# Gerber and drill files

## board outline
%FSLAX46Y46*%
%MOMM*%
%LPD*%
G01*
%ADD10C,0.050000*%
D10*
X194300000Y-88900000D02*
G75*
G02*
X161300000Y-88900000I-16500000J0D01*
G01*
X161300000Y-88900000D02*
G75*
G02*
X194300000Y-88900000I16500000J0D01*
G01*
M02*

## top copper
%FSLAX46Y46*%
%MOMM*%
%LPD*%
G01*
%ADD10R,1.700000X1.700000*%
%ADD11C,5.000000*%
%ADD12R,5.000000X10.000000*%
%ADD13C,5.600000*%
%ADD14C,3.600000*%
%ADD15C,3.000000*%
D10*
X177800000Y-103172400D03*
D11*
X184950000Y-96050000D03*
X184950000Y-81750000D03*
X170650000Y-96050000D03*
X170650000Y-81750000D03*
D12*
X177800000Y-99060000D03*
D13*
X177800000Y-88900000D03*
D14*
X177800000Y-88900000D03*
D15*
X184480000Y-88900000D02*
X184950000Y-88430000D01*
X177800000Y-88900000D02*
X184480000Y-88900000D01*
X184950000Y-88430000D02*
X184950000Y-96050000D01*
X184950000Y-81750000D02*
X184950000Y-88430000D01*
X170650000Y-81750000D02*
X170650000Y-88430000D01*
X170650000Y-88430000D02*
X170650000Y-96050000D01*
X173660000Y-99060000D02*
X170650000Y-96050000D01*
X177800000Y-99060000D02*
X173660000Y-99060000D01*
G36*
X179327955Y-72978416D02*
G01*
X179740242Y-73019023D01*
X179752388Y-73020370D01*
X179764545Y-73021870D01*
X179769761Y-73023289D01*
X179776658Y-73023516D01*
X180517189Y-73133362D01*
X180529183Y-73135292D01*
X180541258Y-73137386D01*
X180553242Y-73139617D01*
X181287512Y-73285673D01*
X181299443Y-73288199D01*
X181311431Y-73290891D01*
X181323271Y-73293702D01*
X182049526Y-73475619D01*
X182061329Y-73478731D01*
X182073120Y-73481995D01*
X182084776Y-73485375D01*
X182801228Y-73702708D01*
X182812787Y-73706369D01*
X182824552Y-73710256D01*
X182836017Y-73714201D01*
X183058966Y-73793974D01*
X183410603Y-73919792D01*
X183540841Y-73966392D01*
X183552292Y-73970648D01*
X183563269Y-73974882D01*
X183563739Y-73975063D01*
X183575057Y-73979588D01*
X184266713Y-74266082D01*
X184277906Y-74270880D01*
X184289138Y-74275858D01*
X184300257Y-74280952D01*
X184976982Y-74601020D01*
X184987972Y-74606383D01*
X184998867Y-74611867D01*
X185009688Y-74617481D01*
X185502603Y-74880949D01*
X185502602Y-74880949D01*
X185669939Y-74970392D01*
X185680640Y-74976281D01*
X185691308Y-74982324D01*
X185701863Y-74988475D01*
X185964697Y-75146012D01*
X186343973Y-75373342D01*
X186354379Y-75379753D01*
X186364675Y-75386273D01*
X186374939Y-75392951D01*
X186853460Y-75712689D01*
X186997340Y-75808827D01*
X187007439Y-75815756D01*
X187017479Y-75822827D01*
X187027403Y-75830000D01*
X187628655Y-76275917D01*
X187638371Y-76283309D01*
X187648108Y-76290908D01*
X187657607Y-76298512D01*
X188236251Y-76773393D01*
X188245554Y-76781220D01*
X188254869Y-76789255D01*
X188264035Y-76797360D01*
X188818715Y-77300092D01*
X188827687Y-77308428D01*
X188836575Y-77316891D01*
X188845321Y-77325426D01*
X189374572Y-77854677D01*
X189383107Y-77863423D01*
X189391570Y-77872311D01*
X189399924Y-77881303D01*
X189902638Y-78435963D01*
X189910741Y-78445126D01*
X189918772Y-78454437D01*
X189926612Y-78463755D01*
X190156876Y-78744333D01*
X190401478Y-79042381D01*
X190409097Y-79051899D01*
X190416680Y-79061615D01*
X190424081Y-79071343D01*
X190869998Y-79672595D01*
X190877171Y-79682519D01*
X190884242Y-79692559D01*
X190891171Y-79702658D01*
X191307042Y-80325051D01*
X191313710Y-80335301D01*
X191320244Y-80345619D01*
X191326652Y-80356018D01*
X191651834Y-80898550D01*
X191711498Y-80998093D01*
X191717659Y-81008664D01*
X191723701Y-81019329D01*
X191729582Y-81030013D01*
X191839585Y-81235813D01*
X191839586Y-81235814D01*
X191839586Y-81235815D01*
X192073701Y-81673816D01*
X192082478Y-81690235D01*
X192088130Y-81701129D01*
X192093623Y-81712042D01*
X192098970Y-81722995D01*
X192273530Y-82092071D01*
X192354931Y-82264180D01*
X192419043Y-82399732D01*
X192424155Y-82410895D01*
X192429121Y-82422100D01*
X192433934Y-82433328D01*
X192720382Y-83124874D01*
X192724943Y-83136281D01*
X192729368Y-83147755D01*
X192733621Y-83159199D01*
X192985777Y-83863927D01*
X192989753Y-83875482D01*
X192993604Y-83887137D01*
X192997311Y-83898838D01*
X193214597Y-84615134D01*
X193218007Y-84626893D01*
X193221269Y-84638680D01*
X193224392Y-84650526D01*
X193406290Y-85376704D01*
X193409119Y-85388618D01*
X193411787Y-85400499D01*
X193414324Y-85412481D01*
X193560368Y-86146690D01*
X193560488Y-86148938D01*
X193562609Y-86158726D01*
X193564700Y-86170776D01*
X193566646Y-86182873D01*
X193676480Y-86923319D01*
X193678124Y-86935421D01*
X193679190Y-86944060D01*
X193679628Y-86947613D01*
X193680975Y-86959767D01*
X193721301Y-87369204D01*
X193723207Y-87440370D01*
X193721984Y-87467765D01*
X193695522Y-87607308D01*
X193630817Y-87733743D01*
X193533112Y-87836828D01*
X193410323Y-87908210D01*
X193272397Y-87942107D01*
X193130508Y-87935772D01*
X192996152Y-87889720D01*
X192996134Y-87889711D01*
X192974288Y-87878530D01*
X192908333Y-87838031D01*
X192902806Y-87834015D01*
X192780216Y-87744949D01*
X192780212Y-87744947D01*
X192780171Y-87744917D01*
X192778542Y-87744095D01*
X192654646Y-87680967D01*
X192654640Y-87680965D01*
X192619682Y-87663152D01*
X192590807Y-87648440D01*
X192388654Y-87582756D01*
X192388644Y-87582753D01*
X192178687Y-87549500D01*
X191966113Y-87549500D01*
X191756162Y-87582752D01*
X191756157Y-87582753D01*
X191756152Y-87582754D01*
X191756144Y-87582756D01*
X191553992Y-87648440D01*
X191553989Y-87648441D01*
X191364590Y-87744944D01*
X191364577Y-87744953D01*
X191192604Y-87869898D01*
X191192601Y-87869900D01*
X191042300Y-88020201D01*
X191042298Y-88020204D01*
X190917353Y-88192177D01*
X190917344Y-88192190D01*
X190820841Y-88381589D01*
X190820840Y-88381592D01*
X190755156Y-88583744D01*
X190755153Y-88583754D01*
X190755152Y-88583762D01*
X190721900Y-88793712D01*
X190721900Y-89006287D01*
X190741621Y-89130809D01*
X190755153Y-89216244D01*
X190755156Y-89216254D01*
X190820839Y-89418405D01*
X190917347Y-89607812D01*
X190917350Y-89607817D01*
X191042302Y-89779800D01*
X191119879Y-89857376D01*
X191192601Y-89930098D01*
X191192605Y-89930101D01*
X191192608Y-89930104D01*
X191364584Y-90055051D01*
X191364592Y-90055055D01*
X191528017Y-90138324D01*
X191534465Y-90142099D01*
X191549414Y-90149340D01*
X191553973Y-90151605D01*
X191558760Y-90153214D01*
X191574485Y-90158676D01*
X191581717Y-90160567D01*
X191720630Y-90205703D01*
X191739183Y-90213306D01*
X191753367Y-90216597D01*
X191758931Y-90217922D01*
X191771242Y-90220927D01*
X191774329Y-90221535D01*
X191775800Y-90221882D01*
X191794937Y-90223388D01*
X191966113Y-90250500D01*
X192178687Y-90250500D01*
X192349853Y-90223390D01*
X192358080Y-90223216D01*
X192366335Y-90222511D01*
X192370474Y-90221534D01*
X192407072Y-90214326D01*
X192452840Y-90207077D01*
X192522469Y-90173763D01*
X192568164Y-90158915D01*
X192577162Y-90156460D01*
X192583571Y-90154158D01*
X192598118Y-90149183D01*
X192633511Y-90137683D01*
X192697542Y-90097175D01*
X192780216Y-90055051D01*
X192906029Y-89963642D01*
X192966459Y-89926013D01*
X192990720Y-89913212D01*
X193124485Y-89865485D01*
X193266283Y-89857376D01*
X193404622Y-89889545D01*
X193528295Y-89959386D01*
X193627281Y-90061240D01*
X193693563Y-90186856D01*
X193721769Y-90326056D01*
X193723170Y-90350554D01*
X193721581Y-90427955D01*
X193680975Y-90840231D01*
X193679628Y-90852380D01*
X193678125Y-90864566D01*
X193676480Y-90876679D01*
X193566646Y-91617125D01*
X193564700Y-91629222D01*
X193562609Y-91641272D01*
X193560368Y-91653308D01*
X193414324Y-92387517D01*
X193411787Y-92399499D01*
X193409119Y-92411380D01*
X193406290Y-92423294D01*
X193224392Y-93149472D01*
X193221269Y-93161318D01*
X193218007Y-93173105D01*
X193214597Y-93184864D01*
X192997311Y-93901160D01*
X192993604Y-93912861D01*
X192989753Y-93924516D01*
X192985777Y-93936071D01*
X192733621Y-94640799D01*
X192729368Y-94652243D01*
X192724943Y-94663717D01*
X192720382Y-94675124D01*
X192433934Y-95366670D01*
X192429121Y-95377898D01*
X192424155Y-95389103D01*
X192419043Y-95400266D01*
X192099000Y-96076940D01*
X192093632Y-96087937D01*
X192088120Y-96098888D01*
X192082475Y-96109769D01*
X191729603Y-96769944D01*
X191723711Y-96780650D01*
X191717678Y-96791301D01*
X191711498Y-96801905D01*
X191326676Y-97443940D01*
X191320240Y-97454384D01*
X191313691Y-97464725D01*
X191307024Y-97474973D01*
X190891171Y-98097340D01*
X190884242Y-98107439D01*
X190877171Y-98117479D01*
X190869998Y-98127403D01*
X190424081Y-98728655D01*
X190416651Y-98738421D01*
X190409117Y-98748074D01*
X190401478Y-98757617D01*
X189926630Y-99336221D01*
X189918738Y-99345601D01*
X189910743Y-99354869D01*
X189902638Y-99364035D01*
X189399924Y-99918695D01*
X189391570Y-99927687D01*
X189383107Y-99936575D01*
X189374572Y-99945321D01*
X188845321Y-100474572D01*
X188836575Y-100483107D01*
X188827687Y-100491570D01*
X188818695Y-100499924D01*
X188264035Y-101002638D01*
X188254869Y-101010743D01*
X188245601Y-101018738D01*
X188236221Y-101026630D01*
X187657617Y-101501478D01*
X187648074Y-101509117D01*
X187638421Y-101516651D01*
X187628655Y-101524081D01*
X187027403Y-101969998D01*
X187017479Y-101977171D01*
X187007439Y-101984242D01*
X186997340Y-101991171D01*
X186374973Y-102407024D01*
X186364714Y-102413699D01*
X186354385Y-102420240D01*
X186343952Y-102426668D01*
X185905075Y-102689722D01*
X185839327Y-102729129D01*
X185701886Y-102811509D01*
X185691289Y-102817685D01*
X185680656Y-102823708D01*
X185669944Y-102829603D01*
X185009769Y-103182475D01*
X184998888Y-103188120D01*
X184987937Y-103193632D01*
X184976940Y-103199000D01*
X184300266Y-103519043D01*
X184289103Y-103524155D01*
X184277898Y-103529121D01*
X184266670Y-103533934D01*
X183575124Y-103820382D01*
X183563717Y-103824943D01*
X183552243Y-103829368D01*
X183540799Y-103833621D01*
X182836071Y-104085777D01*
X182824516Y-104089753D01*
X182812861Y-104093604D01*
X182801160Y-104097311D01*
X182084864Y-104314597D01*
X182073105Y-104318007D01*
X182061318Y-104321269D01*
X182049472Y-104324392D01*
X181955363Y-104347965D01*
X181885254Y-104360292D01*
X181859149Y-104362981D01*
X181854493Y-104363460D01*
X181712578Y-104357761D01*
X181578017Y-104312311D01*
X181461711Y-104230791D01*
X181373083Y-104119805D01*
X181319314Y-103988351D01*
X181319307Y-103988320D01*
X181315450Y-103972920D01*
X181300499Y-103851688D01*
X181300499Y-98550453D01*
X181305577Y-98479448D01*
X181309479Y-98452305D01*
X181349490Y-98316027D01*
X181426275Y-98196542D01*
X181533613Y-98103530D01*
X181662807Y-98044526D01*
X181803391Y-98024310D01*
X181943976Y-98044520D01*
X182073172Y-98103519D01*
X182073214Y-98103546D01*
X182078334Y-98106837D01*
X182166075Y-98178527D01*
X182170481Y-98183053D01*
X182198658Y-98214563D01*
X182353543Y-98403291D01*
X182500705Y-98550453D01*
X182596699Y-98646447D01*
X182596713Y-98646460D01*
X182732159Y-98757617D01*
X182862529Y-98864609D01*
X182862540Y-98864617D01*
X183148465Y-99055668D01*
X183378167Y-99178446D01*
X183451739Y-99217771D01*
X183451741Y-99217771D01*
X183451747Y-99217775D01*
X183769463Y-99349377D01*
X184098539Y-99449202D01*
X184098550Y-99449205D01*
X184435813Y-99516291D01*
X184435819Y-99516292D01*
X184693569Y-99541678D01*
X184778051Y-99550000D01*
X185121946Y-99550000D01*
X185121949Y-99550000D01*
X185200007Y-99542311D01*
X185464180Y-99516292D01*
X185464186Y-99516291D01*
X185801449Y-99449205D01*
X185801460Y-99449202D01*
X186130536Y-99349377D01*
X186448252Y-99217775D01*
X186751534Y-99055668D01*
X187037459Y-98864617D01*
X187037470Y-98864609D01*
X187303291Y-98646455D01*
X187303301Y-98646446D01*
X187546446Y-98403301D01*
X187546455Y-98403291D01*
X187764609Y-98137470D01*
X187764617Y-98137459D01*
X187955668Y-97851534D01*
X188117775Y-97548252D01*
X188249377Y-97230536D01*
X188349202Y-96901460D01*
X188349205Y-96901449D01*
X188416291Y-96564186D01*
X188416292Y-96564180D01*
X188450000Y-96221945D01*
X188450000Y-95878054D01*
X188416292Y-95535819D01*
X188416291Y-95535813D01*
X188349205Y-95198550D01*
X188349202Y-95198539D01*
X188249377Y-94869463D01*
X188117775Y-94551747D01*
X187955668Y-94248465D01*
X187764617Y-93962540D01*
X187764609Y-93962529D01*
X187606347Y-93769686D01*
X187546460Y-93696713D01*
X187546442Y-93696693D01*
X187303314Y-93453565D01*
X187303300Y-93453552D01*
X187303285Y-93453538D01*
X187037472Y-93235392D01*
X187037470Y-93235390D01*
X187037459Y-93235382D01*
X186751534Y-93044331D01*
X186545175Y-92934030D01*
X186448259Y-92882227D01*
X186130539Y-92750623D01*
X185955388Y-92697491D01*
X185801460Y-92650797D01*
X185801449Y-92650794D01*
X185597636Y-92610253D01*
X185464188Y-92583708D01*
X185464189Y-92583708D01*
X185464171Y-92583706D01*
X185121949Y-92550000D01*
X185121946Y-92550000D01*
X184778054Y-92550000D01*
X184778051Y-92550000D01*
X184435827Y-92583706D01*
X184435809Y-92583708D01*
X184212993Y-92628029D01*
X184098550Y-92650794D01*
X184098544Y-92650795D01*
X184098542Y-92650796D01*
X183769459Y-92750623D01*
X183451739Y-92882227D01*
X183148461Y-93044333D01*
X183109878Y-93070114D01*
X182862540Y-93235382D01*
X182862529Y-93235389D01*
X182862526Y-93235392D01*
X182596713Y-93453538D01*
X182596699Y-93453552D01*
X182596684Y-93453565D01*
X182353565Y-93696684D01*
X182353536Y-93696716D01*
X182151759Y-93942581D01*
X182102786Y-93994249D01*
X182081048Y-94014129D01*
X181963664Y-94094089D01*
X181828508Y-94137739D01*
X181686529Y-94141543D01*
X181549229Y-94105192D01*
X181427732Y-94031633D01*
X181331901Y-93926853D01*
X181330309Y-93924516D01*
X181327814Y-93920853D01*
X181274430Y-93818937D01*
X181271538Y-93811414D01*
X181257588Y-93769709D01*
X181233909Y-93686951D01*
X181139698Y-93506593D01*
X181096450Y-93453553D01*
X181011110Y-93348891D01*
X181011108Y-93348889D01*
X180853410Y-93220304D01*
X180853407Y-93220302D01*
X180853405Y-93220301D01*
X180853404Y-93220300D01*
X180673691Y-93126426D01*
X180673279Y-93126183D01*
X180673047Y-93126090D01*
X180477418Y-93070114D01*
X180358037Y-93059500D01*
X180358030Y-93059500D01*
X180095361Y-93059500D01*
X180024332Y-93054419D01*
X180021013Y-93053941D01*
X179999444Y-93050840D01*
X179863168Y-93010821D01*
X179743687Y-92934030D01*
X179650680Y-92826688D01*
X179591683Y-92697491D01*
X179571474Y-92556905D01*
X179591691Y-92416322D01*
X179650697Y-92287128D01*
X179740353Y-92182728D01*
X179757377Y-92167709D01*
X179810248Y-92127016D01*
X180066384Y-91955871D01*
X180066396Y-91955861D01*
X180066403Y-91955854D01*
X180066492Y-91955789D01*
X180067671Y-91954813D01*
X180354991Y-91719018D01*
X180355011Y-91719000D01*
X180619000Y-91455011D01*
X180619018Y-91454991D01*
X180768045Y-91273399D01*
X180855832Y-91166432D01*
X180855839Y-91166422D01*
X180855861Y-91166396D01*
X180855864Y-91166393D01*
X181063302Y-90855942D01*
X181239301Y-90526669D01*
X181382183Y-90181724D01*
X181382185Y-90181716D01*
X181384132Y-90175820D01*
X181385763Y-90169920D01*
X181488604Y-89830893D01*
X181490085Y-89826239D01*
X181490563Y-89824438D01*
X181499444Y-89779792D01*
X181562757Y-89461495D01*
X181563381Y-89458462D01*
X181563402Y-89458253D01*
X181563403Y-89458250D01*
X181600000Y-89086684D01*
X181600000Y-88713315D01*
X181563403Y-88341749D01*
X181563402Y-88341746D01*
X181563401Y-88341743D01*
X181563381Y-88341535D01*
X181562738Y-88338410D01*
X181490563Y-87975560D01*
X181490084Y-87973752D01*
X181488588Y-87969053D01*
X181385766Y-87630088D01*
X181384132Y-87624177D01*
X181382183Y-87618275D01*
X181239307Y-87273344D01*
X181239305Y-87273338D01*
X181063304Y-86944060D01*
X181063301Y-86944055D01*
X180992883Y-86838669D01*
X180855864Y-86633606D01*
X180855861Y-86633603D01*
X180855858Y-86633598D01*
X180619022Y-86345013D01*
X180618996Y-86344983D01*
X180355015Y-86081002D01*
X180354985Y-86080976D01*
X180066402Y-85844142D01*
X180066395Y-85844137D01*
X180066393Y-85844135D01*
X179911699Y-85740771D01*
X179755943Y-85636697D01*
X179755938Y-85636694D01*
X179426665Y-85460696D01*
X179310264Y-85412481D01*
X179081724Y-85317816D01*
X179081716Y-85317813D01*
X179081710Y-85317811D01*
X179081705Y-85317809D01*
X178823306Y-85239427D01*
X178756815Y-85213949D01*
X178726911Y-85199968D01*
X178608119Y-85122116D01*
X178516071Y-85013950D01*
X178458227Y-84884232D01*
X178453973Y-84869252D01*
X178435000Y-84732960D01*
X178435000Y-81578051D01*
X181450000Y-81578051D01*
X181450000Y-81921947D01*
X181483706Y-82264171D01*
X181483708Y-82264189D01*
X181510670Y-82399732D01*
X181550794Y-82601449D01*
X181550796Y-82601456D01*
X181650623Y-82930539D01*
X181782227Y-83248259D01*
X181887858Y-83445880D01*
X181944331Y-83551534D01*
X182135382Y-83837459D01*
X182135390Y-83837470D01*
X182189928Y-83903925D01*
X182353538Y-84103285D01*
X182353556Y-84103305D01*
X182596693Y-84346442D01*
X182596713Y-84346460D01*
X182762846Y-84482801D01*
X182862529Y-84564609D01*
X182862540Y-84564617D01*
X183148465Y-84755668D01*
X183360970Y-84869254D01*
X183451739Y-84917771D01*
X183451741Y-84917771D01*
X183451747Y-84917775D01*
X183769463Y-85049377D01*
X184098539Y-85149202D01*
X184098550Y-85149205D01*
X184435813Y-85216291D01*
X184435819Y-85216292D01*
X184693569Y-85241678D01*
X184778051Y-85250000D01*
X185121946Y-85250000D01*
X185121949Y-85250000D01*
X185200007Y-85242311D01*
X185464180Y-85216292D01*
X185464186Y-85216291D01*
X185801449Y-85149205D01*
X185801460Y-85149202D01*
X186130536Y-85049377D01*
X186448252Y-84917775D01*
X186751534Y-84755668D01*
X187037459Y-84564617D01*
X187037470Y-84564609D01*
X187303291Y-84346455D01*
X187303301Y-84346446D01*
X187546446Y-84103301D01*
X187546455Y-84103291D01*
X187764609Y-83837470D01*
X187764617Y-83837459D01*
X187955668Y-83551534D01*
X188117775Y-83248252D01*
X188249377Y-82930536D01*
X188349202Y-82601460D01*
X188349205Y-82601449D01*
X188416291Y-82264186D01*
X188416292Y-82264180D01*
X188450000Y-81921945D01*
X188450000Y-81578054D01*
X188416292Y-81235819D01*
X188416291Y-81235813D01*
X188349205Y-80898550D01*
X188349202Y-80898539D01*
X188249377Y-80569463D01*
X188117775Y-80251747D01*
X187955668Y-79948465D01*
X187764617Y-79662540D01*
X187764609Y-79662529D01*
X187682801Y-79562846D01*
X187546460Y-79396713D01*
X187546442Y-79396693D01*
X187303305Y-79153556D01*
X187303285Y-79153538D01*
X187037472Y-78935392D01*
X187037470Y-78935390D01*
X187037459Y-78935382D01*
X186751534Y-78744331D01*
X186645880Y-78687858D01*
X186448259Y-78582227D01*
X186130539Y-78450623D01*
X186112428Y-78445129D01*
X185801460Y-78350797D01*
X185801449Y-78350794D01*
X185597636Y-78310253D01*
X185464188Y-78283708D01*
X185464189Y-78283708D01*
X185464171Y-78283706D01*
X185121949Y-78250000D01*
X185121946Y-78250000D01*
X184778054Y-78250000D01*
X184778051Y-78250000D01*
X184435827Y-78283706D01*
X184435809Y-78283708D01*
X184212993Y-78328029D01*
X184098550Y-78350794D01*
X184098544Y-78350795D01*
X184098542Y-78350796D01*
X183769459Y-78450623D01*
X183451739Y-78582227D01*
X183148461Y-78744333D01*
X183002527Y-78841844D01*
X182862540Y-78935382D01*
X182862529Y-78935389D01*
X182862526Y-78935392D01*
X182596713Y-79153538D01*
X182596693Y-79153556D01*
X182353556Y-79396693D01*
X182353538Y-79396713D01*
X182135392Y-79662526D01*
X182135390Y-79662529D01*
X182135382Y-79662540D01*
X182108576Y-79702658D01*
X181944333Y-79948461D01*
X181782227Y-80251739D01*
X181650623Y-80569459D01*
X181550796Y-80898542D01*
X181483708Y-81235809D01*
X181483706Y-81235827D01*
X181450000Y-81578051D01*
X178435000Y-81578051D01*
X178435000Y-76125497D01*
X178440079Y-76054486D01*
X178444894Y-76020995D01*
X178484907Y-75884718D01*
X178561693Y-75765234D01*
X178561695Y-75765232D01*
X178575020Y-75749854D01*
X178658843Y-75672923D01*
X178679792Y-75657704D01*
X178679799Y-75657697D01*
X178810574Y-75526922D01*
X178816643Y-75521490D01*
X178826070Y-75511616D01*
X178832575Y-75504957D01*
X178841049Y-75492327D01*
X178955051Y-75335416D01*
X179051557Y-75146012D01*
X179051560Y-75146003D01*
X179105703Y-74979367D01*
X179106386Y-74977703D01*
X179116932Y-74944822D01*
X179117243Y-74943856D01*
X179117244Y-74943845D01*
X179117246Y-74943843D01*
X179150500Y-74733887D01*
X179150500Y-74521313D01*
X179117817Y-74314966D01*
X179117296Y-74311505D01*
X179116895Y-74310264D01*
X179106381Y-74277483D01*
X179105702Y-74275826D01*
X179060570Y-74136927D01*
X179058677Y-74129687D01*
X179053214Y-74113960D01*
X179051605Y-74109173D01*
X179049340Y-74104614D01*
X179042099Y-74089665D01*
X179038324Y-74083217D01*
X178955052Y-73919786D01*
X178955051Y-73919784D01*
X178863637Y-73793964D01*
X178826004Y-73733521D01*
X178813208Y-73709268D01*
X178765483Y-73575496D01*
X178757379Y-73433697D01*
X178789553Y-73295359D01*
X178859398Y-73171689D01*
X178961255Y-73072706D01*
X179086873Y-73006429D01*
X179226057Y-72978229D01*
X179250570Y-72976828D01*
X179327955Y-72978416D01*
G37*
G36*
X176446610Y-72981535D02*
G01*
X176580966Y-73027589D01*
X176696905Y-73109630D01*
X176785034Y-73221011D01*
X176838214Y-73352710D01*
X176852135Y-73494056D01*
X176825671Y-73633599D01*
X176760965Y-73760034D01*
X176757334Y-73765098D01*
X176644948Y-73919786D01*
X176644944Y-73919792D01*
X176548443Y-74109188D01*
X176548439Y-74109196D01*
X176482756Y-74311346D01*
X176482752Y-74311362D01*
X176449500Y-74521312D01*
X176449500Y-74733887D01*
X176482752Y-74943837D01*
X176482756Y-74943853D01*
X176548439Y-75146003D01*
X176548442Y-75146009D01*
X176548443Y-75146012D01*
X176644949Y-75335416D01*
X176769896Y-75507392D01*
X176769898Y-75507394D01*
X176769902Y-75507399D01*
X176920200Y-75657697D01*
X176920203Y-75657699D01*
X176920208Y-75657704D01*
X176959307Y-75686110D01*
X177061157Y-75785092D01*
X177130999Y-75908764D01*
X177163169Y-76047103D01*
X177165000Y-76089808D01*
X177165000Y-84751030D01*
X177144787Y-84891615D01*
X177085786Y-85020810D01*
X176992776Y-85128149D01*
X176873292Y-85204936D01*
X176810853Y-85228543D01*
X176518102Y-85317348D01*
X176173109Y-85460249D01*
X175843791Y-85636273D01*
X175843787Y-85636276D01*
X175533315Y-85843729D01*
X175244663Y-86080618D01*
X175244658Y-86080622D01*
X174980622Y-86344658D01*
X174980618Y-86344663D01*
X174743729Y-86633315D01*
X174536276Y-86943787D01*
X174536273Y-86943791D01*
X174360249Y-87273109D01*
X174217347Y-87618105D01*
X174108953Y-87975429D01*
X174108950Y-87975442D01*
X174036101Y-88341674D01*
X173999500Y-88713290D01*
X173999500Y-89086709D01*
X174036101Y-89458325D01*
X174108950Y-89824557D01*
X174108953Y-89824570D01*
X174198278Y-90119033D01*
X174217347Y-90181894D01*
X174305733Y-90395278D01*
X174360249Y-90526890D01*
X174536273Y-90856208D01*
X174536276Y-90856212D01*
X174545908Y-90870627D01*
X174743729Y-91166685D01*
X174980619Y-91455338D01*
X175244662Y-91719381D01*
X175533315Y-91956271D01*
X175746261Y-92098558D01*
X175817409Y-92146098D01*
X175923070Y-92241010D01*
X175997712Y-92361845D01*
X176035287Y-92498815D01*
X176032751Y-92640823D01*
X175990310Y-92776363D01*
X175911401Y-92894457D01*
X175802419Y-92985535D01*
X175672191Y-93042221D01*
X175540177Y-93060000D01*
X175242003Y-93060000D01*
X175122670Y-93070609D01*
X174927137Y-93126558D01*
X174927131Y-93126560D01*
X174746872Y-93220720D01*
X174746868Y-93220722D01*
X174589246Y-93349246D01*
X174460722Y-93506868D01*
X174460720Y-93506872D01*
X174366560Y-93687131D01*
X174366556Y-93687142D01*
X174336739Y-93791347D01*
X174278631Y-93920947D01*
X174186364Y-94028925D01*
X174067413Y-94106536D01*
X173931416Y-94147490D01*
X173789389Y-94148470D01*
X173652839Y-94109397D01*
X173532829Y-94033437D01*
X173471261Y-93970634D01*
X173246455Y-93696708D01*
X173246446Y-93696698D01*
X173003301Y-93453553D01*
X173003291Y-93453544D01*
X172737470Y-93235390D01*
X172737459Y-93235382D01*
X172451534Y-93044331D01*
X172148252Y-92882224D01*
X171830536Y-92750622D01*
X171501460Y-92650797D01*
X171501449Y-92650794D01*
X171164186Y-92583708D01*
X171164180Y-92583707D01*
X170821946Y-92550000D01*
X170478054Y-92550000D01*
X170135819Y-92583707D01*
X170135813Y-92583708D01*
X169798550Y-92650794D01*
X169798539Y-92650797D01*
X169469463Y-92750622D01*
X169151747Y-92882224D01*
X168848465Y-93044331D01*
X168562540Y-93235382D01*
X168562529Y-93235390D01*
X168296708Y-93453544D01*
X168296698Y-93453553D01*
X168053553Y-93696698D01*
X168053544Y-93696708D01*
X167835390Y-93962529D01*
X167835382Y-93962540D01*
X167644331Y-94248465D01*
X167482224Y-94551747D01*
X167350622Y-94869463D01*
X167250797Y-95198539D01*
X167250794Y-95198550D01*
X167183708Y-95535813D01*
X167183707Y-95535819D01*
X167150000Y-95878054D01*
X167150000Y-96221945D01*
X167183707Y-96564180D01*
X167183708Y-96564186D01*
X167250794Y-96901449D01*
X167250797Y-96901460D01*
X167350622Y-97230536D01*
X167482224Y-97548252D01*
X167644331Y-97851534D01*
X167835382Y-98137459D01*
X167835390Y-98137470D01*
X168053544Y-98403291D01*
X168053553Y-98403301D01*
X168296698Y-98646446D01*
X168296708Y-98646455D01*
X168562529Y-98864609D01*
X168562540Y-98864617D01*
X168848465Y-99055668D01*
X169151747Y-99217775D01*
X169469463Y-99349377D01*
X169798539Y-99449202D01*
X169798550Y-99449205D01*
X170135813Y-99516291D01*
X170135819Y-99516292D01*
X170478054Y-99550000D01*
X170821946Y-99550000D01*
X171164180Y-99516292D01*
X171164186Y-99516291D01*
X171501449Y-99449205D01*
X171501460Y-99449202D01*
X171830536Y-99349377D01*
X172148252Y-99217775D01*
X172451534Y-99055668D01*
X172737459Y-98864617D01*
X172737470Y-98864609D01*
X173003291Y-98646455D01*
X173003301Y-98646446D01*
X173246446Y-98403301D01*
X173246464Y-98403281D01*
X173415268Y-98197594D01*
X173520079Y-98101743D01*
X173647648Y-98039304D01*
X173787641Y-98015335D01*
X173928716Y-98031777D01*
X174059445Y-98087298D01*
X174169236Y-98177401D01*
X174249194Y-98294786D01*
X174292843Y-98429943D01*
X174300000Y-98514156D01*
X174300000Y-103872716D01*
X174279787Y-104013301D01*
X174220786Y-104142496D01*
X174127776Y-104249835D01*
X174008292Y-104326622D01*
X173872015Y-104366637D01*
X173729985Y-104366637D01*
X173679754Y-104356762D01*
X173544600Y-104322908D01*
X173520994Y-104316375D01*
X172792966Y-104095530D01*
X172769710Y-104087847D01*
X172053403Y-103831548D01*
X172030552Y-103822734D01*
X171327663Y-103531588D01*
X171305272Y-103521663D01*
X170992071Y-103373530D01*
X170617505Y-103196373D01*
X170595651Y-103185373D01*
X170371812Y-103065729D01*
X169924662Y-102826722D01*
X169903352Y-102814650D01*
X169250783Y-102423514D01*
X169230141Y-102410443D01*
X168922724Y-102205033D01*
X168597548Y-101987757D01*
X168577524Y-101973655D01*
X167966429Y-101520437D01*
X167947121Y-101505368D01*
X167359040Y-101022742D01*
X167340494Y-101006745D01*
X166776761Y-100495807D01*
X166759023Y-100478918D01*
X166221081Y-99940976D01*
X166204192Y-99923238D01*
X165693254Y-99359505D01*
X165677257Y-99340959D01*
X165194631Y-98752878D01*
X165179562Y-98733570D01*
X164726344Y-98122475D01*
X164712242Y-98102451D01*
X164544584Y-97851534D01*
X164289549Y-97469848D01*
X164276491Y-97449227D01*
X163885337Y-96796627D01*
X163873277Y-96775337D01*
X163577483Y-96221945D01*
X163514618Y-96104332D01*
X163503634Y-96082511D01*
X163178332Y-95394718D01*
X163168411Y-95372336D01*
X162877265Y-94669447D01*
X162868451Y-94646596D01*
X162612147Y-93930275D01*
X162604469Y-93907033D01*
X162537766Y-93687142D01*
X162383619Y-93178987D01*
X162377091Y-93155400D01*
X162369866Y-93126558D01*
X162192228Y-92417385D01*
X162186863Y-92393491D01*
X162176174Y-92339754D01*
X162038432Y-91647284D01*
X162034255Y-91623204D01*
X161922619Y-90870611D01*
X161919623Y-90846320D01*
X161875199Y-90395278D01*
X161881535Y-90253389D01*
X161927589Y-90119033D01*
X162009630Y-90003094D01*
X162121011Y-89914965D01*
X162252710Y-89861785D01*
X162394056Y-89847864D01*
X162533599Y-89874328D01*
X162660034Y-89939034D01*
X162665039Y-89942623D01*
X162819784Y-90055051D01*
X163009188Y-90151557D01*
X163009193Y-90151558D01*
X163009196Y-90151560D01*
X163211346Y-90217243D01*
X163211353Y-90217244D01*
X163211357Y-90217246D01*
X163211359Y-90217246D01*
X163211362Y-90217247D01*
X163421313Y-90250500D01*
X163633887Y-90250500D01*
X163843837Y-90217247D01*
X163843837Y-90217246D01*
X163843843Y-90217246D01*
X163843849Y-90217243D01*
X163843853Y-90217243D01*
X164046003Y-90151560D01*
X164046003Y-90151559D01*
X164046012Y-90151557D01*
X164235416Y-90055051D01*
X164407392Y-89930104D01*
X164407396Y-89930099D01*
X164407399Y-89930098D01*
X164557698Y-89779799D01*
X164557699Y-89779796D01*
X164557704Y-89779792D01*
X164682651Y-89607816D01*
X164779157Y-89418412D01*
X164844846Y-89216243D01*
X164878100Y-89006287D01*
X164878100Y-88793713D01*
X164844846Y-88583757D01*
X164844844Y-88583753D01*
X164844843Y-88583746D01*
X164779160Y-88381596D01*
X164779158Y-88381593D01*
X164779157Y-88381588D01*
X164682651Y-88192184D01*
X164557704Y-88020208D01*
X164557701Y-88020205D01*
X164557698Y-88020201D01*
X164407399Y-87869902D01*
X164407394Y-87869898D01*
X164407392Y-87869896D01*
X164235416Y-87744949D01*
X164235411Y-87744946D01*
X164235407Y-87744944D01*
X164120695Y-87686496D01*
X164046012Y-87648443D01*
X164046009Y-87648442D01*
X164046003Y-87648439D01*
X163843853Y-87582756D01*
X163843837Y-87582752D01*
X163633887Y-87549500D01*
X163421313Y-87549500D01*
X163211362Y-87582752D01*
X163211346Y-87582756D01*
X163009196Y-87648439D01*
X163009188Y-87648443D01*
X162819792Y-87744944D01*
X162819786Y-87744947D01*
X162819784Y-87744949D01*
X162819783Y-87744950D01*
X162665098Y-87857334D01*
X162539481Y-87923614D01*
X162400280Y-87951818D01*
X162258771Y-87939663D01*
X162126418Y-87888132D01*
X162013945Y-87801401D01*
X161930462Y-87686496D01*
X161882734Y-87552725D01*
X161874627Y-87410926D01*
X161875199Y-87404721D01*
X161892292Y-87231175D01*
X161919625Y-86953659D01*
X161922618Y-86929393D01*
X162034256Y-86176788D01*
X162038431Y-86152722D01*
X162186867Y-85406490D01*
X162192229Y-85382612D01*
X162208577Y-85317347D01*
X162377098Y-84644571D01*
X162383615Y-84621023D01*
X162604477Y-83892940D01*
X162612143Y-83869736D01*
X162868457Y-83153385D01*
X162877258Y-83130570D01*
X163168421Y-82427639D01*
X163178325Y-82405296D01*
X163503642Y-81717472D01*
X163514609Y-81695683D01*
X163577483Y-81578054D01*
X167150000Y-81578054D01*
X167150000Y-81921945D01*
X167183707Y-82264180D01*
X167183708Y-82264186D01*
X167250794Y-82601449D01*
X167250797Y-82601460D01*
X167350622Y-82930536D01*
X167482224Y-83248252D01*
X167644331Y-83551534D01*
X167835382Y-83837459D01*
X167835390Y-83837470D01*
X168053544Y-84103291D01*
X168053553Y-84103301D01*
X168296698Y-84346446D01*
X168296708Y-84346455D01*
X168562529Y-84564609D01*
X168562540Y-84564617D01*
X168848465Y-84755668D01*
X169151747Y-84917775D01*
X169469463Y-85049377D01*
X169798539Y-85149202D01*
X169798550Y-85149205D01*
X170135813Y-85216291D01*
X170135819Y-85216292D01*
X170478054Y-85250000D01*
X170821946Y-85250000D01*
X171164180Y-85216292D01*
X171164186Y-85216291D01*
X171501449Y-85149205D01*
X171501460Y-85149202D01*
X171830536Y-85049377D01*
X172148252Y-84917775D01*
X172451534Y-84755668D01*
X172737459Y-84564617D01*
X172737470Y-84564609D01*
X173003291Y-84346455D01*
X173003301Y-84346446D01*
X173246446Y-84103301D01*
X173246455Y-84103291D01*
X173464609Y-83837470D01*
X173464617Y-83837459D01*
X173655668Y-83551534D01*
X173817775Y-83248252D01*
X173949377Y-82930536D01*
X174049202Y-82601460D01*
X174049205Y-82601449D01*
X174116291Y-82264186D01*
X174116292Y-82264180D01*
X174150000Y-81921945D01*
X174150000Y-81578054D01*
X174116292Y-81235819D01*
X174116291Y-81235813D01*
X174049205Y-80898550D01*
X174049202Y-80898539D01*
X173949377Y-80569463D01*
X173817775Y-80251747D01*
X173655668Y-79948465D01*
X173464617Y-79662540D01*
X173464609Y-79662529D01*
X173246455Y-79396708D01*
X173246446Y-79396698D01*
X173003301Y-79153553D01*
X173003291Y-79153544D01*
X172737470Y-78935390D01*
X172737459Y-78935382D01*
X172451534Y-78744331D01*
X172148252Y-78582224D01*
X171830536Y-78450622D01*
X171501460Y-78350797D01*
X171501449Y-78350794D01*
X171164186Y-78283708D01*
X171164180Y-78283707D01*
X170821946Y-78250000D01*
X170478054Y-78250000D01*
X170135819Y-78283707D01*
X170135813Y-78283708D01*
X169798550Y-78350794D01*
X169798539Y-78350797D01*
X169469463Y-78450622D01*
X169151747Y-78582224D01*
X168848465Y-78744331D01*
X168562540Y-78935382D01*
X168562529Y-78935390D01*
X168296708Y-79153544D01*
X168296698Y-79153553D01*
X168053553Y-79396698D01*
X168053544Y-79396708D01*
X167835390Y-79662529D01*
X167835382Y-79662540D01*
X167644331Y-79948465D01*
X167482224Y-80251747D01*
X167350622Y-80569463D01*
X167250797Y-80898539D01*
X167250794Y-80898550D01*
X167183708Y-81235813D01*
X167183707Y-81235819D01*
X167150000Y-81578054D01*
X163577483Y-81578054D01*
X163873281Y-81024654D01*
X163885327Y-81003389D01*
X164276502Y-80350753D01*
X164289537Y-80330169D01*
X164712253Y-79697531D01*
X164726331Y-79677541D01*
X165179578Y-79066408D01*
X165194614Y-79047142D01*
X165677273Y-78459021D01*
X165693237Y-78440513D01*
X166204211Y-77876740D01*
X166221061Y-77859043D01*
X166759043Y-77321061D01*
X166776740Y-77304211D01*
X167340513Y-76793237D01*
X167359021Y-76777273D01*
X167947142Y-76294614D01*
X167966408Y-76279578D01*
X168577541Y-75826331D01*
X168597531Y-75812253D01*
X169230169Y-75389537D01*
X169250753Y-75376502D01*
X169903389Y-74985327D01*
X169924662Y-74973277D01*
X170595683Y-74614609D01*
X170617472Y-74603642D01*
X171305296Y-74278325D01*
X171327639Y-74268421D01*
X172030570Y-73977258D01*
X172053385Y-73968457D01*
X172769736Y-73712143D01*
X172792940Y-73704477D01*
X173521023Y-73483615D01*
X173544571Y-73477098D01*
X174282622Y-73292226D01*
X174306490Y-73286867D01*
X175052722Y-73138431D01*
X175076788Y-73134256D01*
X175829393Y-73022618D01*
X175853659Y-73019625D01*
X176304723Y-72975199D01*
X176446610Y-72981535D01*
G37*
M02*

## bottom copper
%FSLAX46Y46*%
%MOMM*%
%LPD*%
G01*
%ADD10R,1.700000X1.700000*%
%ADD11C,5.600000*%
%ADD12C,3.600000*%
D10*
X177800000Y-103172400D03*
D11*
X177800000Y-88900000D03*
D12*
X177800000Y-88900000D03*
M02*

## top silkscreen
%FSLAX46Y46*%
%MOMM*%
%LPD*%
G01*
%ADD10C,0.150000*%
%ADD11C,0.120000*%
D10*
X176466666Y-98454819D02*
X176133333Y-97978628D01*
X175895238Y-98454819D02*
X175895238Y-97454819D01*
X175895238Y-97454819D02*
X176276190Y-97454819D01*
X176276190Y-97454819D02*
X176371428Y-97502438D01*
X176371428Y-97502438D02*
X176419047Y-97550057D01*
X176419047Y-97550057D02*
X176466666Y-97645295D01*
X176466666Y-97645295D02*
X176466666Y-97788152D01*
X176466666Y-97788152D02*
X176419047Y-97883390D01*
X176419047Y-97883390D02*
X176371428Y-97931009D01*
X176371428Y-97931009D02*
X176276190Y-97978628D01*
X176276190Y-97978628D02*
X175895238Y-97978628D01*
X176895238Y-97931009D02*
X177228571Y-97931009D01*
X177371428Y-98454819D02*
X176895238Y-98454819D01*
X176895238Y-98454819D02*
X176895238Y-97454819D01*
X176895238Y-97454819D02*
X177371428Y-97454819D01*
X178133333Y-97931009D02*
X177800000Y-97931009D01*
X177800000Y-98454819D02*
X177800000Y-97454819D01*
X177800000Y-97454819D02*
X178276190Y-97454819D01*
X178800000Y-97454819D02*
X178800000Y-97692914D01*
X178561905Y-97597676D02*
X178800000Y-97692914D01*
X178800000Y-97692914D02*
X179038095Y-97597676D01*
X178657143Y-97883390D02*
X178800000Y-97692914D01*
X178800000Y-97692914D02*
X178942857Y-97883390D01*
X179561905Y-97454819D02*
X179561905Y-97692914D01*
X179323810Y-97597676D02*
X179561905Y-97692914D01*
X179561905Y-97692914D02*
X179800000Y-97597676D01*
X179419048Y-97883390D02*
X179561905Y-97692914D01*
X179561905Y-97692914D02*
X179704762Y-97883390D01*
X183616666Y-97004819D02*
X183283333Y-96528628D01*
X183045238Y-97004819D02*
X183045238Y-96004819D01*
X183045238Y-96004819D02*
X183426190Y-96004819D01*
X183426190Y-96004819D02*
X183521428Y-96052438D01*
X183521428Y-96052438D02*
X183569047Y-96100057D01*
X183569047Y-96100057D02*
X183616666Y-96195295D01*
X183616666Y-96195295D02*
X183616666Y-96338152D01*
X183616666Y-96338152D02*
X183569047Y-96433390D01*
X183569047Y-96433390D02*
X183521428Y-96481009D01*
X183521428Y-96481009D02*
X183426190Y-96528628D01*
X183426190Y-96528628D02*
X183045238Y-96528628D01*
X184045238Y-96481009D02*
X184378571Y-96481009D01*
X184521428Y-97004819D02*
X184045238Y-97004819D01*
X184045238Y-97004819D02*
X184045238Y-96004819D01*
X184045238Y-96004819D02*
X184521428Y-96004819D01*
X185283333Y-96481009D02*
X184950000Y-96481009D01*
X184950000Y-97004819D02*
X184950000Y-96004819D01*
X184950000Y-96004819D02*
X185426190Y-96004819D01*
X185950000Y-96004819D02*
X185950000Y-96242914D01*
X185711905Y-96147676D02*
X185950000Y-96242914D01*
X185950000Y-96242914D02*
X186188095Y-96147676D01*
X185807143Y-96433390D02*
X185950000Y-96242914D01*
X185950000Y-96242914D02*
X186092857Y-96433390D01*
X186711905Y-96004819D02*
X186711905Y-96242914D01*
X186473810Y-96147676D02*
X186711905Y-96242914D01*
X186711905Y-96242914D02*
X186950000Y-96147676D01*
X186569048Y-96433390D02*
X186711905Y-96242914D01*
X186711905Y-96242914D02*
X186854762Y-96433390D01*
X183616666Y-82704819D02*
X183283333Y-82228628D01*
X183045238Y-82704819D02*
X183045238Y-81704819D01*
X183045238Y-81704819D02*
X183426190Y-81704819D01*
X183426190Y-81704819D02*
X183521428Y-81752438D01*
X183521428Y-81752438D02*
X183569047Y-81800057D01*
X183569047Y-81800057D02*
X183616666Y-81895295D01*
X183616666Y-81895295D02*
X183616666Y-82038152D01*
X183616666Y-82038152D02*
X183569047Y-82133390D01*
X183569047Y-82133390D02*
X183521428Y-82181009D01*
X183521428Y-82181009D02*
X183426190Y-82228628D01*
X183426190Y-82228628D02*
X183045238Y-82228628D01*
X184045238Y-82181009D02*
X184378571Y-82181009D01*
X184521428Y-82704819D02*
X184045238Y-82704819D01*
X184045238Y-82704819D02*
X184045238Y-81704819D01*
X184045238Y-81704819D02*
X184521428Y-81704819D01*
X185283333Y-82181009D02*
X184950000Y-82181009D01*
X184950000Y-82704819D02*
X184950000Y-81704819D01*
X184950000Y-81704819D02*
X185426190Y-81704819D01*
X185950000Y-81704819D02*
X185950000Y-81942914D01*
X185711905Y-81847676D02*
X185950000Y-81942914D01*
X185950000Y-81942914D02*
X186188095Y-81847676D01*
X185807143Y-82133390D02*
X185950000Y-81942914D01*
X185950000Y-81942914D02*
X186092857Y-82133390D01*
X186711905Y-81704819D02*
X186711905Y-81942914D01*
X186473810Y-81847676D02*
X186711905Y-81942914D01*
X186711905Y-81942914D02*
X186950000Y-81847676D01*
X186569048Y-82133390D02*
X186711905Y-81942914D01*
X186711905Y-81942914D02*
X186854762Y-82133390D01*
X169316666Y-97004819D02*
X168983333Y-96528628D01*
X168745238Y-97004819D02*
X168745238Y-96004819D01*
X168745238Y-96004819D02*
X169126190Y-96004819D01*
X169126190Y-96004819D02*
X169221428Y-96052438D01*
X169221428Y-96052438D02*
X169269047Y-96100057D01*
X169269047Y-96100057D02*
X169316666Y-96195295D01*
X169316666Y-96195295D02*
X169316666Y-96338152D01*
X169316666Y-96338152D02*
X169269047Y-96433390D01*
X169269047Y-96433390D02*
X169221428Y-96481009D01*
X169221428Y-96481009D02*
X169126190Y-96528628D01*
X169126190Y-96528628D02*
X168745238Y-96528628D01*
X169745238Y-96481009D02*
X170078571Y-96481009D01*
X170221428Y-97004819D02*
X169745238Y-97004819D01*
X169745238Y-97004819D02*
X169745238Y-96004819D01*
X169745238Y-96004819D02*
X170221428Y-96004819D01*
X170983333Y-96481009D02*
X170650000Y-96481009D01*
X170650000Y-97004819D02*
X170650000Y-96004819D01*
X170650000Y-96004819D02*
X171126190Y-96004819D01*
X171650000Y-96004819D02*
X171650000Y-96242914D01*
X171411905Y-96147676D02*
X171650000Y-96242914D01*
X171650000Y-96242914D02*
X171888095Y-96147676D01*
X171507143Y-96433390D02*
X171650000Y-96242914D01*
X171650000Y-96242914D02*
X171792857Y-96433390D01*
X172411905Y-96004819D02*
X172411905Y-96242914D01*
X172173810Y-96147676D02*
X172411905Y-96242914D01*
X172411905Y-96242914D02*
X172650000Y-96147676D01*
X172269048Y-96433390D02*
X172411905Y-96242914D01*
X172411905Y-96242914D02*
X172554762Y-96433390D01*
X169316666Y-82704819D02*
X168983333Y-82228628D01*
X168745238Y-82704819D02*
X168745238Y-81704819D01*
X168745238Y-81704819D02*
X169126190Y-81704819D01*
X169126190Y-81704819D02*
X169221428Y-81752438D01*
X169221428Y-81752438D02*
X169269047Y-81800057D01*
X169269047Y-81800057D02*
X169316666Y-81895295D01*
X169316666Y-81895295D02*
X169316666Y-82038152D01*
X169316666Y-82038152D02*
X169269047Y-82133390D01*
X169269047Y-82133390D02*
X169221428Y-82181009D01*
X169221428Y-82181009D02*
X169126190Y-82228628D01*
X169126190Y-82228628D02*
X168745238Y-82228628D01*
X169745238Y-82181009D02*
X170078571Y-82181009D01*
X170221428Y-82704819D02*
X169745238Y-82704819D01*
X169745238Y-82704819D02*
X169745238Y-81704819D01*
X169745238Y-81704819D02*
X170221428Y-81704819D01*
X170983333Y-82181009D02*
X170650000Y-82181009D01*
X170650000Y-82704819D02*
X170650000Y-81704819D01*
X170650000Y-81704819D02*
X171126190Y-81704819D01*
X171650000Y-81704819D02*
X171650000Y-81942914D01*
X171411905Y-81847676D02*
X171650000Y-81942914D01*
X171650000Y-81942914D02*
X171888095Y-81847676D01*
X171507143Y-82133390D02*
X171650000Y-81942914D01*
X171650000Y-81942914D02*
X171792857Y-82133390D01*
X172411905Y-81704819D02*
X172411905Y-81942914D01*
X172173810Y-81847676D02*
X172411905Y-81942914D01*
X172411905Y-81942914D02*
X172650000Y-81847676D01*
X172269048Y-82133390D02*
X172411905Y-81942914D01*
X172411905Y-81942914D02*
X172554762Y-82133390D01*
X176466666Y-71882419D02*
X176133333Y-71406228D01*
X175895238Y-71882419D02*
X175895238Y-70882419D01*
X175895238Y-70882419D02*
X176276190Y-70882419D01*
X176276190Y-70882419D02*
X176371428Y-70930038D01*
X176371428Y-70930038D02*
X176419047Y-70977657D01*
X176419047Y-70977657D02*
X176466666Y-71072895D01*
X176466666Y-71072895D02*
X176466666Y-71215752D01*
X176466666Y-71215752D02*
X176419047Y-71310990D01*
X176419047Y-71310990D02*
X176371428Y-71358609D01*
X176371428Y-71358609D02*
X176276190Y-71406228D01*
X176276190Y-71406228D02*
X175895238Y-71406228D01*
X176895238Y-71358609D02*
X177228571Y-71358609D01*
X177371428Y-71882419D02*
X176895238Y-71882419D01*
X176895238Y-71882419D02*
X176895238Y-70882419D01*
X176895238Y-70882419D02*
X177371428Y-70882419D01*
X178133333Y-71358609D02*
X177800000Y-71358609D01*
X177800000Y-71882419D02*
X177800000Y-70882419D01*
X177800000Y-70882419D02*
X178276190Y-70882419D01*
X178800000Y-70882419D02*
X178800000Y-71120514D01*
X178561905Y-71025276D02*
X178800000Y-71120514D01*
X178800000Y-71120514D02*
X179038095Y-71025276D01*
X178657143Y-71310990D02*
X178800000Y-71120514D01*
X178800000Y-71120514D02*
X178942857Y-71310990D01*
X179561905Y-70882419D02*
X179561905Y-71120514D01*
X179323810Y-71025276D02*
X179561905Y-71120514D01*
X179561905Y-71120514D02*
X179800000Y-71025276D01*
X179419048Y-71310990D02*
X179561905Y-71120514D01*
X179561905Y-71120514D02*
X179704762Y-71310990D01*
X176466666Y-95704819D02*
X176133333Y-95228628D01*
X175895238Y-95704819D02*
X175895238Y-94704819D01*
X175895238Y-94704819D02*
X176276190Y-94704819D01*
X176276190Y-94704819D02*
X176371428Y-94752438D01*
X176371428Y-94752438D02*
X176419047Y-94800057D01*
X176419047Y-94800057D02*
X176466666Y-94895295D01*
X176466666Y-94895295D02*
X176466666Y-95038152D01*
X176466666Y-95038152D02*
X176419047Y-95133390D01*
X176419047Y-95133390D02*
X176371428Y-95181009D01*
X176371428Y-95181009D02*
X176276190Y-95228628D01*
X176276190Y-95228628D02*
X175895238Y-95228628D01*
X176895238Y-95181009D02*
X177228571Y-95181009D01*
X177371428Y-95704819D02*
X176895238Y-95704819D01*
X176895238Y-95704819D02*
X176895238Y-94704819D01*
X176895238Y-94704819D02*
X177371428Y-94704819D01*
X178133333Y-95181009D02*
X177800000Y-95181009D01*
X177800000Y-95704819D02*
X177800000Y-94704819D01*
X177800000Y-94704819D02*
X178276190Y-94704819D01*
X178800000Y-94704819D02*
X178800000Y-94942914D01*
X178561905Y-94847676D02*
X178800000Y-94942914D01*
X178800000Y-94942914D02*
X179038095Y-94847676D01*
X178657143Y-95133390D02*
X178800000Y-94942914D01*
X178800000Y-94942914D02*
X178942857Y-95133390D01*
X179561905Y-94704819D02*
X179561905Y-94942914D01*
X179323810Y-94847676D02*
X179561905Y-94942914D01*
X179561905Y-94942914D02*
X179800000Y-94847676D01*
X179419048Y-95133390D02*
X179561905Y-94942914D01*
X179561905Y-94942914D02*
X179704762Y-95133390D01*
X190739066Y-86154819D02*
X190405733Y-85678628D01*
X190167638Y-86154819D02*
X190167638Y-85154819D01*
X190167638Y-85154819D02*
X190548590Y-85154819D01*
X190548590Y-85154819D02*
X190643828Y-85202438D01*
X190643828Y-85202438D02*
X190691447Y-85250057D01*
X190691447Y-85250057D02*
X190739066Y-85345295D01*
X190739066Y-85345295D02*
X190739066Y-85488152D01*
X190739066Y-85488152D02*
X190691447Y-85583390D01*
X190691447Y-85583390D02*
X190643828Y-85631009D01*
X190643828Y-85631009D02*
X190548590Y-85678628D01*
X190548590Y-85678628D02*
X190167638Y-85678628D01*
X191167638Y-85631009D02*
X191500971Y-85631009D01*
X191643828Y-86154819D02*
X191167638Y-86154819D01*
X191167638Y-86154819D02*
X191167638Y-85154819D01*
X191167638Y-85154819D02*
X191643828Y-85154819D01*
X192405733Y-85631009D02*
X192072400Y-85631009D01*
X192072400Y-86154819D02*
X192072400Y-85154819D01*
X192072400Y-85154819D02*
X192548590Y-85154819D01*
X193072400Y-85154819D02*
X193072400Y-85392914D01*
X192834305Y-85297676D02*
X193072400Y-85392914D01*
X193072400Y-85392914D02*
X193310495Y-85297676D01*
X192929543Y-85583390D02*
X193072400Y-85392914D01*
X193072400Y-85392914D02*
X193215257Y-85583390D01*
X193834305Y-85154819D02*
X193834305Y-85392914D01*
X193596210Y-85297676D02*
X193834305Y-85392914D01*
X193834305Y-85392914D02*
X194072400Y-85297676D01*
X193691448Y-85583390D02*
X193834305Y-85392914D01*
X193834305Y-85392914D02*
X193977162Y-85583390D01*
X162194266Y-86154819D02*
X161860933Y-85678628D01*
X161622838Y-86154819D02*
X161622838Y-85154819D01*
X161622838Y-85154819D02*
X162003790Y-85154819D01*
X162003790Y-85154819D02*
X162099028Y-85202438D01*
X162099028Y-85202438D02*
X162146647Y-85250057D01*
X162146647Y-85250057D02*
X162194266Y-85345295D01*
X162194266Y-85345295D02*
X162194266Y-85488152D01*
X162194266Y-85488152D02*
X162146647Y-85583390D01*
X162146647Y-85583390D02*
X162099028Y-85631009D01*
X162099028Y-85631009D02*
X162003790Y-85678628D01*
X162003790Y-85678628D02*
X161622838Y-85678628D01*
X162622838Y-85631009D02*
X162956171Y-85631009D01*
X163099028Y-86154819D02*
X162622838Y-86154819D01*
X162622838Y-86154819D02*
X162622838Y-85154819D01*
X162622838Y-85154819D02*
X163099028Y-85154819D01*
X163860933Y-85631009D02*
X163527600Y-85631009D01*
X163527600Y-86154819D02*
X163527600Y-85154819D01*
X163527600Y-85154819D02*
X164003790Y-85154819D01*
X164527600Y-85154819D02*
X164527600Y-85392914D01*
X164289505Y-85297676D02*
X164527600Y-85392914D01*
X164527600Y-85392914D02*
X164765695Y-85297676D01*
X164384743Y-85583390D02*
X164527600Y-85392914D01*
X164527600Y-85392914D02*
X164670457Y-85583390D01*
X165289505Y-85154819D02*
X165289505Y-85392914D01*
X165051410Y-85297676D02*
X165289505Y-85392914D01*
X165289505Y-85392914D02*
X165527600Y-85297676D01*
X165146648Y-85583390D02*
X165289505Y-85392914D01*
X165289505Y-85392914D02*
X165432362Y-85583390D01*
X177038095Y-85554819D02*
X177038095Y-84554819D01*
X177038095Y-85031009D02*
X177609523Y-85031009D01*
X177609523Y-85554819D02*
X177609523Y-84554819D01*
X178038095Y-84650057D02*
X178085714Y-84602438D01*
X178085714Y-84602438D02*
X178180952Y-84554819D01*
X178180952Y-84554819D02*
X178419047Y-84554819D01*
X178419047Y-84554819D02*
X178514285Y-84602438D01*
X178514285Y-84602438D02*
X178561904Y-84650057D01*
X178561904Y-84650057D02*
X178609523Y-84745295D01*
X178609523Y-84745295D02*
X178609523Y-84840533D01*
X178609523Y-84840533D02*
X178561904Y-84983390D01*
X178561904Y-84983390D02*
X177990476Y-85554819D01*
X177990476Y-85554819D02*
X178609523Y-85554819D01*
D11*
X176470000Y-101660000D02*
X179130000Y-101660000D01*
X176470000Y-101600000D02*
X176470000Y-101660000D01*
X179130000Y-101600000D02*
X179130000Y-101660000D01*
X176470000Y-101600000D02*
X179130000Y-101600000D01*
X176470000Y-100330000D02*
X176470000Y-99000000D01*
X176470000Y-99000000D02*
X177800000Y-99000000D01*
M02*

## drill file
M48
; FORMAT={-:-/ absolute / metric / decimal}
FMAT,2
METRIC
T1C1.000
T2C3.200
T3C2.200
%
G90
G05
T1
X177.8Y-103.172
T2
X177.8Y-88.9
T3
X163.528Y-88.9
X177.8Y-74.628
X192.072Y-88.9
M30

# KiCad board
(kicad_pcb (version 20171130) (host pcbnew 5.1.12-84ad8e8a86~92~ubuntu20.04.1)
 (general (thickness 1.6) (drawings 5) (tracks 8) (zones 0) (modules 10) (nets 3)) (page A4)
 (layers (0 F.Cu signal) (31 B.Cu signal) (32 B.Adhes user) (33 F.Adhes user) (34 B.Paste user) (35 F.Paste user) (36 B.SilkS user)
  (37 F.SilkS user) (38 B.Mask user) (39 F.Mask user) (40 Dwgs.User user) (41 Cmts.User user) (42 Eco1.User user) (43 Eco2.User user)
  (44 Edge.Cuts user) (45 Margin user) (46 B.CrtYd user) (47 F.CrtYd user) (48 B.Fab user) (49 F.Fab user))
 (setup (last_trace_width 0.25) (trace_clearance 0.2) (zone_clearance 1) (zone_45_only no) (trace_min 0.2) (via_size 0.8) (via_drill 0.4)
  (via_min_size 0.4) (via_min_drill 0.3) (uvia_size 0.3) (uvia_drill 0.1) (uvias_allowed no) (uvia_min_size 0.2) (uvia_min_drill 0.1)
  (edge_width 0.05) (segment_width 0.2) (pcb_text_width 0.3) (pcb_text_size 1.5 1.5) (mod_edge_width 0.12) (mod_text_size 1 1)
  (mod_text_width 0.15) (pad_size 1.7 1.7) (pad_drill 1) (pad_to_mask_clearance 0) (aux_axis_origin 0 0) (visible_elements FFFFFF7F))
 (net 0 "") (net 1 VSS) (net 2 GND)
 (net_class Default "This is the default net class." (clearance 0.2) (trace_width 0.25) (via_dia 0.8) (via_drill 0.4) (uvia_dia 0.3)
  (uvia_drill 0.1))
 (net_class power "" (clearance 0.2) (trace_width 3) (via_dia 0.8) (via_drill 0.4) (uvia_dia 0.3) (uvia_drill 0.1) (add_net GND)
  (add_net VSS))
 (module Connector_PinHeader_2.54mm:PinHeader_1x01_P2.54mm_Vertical (layer F.Cu) (at 177.8 100.33)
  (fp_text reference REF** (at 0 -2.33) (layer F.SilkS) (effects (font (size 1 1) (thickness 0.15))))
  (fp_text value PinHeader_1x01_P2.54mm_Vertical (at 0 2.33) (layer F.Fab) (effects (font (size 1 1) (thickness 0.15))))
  (fp_line (start -1.33 1.33) (end 1.33 1.33) (layer F.SilkS) (width 0.12))
  (fp_line (start -1.33 1.27) (end -1.33 1.33) (layer F.SilkS) (width 0.12))
  (fp_line (start 1.33 1.27) (end 1.33 1.33) (layer F.SilkS) (width 0.12))
  (fp_line (start -1.33 1.27) (end 1.33 1.27) (layer F.SilkS) (width 0.12))
  (fp_line (start -1.33 0) (end -1.33 -1.33) (layer F.SilkS) (width 0.12))
  (fp_line (start -1.33 -1.33) (end 0 -1.33) (layer F.SilkS) (width 0.12))
  (pad 1 thru_hole rect (at 0 2.8424) (size 1.7 1.7) (drill 1) (layers *.Cu *.Mask) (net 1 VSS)))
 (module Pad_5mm (layer F.Cu) (at 184.95 96.05)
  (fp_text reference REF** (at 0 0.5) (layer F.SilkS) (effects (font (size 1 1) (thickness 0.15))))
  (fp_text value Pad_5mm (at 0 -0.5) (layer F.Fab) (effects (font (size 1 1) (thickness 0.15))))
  (pad 1 smd circle (at 0 0) (size 5 5) (layers F.Cu F.Paste F.Mask) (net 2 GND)))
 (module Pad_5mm (layer F.Cu) (at 184.95 81.75)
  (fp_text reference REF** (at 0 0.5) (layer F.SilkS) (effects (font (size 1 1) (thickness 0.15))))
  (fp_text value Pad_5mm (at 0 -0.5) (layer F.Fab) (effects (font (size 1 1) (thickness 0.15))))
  (pad 1 smd circle (at 0 0) (size 5 5) (layers F.Cu F.Paste F.Mask) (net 2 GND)))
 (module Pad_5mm (layer F.Cu) (at 170.65 96.05)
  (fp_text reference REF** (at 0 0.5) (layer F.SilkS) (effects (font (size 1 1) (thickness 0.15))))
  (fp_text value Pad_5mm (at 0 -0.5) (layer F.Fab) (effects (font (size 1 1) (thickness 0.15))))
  (pad 1 smd circle (at 0 0) (size 5 5) (layers F.Cu F.Paste F.Mask) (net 1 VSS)))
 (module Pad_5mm (layer F.Cu) (at 170.65 81.75)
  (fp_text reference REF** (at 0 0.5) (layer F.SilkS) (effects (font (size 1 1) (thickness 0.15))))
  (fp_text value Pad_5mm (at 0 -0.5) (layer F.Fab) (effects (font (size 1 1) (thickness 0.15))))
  (pad 1 smd circle (at 0 0) (size 5 5) (layers F.Cu F.Paste F.Mask) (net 1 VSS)))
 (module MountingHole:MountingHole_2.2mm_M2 (layer F.Cu) (at 177.8 74.6276)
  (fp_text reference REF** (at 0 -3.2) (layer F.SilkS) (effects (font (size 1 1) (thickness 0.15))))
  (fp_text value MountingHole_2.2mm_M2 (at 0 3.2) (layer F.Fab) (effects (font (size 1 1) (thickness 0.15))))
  (pad 1 np_thru_hole circle (at 0 0) (size 2.2 2.2) (drill 2.2) (layers *.Cu *.Mask)))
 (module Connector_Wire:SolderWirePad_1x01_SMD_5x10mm (layer F.Cu) (at 177.8 99.06)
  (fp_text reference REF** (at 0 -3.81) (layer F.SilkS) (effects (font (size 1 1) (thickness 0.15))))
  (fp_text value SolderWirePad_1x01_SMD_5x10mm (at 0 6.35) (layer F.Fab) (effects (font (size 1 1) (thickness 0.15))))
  (pad 1 smd rect (at 0 0) (size 5 10) (layers F.Cu F.Paste F.Mask) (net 1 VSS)))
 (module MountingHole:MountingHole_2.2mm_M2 (layer F.Cu) (at 192.0724 88.9)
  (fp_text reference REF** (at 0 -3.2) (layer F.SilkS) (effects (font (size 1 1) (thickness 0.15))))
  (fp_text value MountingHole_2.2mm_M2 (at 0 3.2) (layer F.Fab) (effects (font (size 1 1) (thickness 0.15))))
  (pad 1 np_thru_hole circle (at 0 0) (size 2.2 2.2) (drill 2.2) (layers *.Cu *.Mask)))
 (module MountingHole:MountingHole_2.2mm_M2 (layer F.Cu) (at 163.5276 88.9)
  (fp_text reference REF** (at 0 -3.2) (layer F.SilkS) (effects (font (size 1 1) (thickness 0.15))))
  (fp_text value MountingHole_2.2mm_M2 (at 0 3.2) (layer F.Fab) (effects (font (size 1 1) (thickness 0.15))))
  (pad 1 np_thru_hole circle (at 0 0) (size 2.2 2.2) (drill 2.2) (layers *.Cu *.Mask)))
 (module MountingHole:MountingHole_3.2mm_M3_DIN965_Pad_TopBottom (layer F.Cu) (at 177.8 88.9)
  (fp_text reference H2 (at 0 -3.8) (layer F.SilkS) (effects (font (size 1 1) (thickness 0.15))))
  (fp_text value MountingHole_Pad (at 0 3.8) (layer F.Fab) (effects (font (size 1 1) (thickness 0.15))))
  (pad 1 connect circle (at 0 0) (size 5.6 5.6) (layers B.Cu B.Mask) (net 2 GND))
  (pad 1 connect circle (at 0 0) (size 5.6 5.6) (layers F.Cu F.Mask) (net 2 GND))
  (pad 1 thru_hole circle (at 0 0) (size 3.6 3.6) (drill 3.2) (layers *.Cu *.Mask) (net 2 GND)))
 (gr_circle (center 177.8 88.9) (end 194.3 88.9) (layer Edge.Cuts) (width 0.05))
 (segment (start 184.48 88.9) (end 184.95 88.43) (width 3) (layer F.Cu) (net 2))
 (segment (start 177.8 88.9) (end 184.48 88.9) (width 3) (layer F.Cu) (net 2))
 (segment (start 184.95 88.43) (end 184.95 96.05) (width 3) (layer F.Cu) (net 2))
 (segment (start 184.95 81.75) (end 184.95 88.43) (width 3) (layer F.Cu) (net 2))
 (segment (start 170.65 81.75) (end 170.65 88.43) (width 3) (layer F.Cu) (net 1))
 (segment (start 170.65 88.43) (end 170.65 96.05) (width 3) (layer F.Cu) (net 1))
 (segment (start 173.66 99.06) (end 170.65 96.05) (width 3) (layer F.Cu) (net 1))
 (segment (start 177.8 99.06) (end 173.66 99.06) (width 3) (layer F.Cu) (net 1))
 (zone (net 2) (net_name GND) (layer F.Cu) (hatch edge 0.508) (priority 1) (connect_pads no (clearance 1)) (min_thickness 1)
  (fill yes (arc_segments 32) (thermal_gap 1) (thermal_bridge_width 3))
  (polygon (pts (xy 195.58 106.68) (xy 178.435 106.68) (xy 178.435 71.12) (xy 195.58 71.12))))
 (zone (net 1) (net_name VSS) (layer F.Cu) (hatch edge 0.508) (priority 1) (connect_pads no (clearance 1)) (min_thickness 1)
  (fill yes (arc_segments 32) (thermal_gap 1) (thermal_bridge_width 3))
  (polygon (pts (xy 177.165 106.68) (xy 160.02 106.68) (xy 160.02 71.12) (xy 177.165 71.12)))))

